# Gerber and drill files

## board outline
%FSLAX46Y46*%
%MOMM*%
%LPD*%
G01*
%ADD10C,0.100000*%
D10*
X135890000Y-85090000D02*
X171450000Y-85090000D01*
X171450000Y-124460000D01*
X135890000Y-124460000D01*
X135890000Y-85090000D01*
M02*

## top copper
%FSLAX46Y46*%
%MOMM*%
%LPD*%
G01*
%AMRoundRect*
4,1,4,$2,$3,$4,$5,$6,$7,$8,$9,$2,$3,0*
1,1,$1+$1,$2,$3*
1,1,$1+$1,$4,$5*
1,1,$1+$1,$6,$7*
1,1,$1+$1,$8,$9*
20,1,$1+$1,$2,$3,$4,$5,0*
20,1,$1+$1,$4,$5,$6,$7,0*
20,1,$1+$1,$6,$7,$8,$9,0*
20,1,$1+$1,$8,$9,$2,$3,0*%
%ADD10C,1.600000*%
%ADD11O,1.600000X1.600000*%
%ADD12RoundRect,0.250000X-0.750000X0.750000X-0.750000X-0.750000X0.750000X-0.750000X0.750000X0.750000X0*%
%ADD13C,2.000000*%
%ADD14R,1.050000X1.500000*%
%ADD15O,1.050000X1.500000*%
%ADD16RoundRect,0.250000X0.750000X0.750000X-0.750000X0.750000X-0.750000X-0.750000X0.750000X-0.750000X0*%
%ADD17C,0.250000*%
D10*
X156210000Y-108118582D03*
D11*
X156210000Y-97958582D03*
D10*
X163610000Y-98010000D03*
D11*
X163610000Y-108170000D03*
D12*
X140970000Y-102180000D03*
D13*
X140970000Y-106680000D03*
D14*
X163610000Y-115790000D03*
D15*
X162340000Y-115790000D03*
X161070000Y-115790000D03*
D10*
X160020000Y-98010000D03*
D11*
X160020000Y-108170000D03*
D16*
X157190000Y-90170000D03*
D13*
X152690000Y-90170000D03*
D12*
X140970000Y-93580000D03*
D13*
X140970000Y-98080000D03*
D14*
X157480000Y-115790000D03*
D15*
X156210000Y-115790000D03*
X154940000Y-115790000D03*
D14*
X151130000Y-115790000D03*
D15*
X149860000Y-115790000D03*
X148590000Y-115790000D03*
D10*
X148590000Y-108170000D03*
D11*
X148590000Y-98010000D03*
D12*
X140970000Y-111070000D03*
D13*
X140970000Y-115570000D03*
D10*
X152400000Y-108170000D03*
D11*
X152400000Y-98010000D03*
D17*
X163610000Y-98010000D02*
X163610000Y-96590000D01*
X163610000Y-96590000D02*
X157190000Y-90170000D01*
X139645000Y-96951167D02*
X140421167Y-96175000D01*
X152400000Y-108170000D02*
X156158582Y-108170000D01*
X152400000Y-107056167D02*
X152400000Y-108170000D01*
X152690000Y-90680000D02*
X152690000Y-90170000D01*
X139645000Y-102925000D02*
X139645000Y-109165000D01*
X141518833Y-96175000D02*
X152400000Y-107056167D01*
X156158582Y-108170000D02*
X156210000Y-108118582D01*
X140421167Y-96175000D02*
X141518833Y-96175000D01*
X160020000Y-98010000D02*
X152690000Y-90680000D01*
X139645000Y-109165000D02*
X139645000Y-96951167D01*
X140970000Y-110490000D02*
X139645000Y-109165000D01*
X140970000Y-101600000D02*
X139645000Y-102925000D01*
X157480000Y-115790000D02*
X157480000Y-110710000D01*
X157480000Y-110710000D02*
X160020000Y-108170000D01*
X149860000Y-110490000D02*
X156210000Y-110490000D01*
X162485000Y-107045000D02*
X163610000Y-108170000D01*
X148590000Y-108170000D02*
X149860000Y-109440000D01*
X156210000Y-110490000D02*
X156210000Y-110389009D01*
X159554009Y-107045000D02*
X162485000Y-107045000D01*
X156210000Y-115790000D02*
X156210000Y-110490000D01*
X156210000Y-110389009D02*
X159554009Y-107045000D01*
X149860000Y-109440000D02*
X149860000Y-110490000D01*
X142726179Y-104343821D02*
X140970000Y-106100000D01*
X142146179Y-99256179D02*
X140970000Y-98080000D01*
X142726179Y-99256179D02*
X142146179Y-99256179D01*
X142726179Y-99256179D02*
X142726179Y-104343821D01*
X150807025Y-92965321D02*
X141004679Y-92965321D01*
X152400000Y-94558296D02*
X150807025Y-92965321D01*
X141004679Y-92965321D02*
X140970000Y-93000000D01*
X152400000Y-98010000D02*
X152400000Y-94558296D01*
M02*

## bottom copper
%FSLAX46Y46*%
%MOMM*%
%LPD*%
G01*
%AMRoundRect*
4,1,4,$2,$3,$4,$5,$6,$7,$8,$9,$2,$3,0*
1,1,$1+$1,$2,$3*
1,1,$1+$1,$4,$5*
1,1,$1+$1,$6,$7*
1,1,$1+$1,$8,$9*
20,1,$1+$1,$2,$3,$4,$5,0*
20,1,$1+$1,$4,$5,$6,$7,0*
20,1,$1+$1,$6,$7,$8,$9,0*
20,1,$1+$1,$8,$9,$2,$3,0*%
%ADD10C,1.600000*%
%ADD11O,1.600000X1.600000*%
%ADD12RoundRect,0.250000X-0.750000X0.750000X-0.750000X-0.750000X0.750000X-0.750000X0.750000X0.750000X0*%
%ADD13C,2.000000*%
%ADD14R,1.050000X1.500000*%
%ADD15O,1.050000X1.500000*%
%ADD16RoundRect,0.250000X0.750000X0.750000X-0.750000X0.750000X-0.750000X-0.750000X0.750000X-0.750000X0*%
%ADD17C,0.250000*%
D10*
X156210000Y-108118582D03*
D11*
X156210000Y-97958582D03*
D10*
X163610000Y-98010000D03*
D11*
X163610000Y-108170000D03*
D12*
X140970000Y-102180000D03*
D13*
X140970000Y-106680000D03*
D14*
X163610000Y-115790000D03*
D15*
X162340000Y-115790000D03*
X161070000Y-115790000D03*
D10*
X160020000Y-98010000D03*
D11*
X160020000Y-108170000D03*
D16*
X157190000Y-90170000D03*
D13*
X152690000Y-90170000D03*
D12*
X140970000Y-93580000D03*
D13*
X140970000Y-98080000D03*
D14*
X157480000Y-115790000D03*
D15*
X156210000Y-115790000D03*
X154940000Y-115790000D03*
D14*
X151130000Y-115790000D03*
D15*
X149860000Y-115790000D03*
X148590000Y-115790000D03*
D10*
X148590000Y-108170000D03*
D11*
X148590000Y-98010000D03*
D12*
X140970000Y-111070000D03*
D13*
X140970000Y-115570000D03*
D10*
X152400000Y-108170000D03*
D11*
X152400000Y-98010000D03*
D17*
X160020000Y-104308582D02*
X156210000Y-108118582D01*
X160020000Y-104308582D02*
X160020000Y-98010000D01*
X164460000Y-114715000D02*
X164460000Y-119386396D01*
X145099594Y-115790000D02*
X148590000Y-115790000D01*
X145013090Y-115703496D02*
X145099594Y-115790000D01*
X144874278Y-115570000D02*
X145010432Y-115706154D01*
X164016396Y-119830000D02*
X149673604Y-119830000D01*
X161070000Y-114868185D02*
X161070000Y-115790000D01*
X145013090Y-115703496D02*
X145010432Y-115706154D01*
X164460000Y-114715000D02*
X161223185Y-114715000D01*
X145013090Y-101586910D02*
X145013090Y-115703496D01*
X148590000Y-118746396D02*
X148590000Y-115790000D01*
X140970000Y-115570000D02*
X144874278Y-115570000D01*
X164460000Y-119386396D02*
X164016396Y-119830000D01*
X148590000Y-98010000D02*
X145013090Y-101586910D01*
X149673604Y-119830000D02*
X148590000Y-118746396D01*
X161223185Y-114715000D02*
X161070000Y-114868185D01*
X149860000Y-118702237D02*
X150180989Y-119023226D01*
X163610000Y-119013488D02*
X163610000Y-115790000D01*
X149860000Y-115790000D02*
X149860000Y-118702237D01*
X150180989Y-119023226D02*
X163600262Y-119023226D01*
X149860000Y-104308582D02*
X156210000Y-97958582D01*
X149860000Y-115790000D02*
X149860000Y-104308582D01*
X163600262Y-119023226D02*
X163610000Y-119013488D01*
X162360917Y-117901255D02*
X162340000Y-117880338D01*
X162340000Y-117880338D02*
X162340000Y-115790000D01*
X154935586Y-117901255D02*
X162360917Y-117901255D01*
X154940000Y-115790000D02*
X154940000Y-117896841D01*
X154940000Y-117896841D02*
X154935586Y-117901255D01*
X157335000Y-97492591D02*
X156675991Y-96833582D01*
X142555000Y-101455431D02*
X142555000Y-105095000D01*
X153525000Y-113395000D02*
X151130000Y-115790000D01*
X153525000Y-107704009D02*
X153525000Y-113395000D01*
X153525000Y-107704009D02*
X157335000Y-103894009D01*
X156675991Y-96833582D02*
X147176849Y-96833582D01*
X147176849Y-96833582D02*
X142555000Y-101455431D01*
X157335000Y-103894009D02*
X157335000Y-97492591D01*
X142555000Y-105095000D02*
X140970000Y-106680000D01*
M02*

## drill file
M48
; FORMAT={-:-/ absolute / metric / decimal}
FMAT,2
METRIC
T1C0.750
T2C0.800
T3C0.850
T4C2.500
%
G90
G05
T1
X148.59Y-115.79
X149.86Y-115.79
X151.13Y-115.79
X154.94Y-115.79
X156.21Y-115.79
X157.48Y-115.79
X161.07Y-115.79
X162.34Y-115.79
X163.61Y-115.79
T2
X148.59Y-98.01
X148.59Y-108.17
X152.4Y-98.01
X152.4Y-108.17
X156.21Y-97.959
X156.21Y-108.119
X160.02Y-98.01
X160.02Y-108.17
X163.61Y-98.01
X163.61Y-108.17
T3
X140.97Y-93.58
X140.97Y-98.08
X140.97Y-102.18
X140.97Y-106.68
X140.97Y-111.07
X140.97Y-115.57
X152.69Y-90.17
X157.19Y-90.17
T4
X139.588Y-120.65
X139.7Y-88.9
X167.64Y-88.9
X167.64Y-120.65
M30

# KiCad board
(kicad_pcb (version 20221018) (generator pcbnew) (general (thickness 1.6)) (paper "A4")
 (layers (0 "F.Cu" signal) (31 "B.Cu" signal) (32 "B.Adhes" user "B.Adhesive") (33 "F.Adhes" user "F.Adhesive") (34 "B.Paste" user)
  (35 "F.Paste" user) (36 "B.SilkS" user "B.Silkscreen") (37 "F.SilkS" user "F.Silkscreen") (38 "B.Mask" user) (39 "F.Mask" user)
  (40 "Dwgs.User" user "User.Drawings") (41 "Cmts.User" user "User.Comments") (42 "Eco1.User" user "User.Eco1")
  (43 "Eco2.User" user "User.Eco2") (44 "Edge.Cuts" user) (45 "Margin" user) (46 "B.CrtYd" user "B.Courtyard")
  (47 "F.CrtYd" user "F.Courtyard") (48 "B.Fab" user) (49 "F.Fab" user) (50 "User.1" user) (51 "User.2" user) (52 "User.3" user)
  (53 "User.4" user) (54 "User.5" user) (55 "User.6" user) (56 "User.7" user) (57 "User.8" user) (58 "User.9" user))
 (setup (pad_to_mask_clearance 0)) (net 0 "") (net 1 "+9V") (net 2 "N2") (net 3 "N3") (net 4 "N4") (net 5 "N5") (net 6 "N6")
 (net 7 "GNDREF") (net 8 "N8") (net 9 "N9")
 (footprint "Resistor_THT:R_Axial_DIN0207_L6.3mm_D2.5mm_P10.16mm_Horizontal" (layer "F.Cu") (at 156.21 108.118582 90)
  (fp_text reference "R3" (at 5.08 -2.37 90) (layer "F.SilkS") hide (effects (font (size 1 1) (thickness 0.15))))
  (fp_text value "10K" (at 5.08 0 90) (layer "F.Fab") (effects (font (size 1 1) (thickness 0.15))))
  (pad "1" thru_hole circle (at 0 0 90) (size 1.6 1.6) (drill 0.8) (layers "*.Cu" "*.Mask") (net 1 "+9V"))
  (pad "2" thru_hole oval (at 10.16 0 90) (size 1.6 1.6) (drill 0.8) (layers "*.Cu" "*.Mask") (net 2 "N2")))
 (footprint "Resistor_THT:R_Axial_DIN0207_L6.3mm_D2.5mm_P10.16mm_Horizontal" (layer "F.Cu") (at 163.61 98.01 -90)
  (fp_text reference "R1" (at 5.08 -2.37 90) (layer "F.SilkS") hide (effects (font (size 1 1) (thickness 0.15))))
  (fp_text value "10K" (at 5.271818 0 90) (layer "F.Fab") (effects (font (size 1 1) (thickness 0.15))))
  (pad "1" thru_hole circle (at 0 0 270) (size 1.6 1.6) (drill 0.8) (layers "*.Cu" "*.Mask") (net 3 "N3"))
  (pad "2" thru_hole oval (at 10.16 0 270) (size 1.6 1.6) (drill 0.8) (layers "*.Cu" "*.Mask") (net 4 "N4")))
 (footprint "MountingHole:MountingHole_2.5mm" (layer "F.Cu") (at 139.7 88.9)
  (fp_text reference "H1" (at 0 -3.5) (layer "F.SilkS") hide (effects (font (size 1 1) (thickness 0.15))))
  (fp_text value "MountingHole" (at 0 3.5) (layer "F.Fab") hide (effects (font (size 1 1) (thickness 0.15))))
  (pad "" np_thru_hole circle (at 0 0) (size 2.5 2.5) (drill 2.5) (layers "*.Cu" "*.Mask")))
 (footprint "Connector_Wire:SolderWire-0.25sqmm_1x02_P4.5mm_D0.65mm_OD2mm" (layer "F.Cu") (at 140.97 102.18 -90)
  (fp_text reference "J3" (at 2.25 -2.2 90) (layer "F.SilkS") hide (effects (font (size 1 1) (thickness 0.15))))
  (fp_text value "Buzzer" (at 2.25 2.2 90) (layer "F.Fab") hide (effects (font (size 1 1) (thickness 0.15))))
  (pad "1" thru_hole roundrect (at 0 0 270) (size 2 2) (drill 0.85) (layers "*.Cu" "*.Mask") (roundrect_rratio 0.125) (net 1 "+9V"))
  (pad "2" thru_hole circle (at 4.5 0 270) (size 2 2) (drill 0.85) (layers "*.Cu" "*.Mask") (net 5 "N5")))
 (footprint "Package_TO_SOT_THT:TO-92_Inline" (layer "F.Cu") (at 163.61 115.79 180)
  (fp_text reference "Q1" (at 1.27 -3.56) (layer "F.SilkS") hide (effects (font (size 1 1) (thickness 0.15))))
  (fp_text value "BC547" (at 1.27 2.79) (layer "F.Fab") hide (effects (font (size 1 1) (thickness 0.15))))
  (pad "1" thru_hole rect (at 0 0 180) (size 1.05 1.5) (drill 0.75) (layers "*.Cu" "*.Mask") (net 2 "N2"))
  (pad "2" thru_hole oval (at 1.27 0 180) (size 1.05 1.5) (drill 0.75) (layers "*.Cu" "*.Mask") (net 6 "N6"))
  (pad "3" thru_hole oval (at 2.54 0 180) (size 1.05 1.5) (drill 0.75) (layers "*.Cu" "*.Mask") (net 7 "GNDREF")))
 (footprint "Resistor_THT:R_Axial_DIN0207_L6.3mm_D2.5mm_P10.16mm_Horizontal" (layer "F.Cu") (at 160.02 98.01 -90)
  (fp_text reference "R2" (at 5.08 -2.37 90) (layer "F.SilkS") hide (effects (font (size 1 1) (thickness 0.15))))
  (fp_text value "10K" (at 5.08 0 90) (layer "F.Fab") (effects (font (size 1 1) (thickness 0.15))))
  (pad "1" thru_hole circle (at 0 0 270) (size 1.6 1.6) (drill 0.8) (layers "*.Cu" "*.Mask") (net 1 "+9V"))
  (pad "2" thru_hole oval (at 10.16 0 270) (size 1.6 1.6) (drill 0.8) (layers "*.Cu" "*.Mask") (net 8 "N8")))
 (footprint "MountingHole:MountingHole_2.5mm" (layer "F.Cu") (at 139.588015 120.65)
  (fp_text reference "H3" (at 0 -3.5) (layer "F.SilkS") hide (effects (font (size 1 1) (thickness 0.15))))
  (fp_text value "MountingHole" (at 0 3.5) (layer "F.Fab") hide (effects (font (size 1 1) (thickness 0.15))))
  (pad "" np_thru_hole circle (at 0 0) (size 2.5 2.5) (drill 2.5) (layers "*.Cu" "*.Mask")))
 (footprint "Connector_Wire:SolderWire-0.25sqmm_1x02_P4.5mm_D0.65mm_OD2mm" (layer "F.Cu") (at 157.19 90.17 180)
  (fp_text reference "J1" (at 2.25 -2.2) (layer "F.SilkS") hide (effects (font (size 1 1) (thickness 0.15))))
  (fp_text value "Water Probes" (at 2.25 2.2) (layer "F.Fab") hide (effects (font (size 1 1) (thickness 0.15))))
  (pad "1" thru_hole roundrect (at 0 0 180) (size 2 2) (drill 0.85) (layers "*.Cu" "*.Mask") (roundrect_rratio 0.125) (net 3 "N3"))
  (pad "2" thru_hole circle (at 4.5 0 180) (size 2 2) (drill 0.85) (layers "*.Cu" "*.Mask") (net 1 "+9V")))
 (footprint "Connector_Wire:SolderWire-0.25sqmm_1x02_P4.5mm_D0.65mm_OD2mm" (layer "F.Cu") (at 140.97 93.58 -90)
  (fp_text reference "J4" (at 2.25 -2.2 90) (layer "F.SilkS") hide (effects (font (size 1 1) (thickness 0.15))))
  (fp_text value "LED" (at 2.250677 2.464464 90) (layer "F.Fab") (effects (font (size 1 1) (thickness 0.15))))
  (pad "1" thru_hole roundrect (at 0 0 270) (size 2 2) (drill 0.85) (layers "*.Cu" "*.Mask") (roundrect_rratio 0.125) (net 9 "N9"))
  (pad "2" thru_hole circle (at 4.5 0 270) (size 2 2) (drill 0.85) (layers "*.Cu" "*.Mask") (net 5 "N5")))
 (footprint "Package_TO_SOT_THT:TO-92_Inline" (layer "F.Cu") (at 157.48 115.79 180)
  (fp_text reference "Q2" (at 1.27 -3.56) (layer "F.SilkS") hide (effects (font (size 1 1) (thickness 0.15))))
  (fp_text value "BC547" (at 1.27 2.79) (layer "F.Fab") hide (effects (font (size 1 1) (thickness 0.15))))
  (pad "1" thru_hole rect (at 0 0 180) (size 1.05 1.5) (drill 0.75) (layers "*.Cu" "*.Mask") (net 8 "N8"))
  (pad "2" thru_hole oval (at 1.27 0 180) (size 1.05 1.5) (drill 0.75) (layers "*.Cu" "*.Mask") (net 4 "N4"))
  (pad "3" thru_hole oval (at 2.54 0 180) (size 1.05 1.5) (drill 0.75) (layers "*.Cu" "*.Mask") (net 6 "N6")))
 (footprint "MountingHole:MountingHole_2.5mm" (layer "F.Cu") (at 167.64 120.65)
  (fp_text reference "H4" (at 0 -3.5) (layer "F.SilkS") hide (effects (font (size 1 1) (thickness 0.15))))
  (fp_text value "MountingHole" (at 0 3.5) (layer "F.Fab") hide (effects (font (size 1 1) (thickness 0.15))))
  (pad "" np_thru_hole circle (at 0 0) (size 2.5 2.5) (drill 2.5) (layers "*.Cu" "*.Mask")))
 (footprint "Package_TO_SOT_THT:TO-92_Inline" (layer "F.Cu") (at 151.13 115.79 180)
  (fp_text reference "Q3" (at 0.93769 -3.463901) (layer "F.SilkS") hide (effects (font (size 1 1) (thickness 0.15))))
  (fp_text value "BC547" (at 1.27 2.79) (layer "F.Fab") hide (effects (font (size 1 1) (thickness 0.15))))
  (pad "1" thru_hole rect (at 0 0 180) (size 1.05 1.5) (drill 0.75) (layers "*.Cu" "*.Mask") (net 5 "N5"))
  (pad "2" thru_hole oval (at 1.27 0 180) (size 1.05 1.5) (drill 0.75) (layers "*.Cu" "*.Mask") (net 2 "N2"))
  (pad "3" thru_hole oval (at 2.54 0 180) (size 1.05 1.5) (drill 0.75) (layers "*.Cu" "*.Mask") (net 7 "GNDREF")))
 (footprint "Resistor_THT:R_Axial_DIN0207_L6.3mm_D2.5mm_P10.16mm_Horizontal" (layer "F.Cu") (at 148.59 108.17 90)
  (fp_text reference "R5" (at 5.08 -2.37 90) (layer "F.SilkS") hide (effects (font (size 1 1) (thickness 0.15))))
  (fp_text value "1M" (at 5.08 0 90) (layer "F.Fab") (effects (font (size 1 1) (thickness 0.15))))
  (pad "1" thru_hole circle (at 0 0 90) (size 1.6 1.6) (drill 0.8) (layers "*.Cu" "*.Mask") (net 4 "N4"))
  (pad "2" thru_hole oval (at 10.16 0 90) (size 1.6 1.6) (drill 0.8) (layers "*.Cu" "*.Mask") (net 7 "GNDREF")))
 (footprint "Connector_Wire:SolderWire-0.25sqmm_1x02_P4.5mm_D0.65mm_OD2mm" (layer "F.Cu") (at 140.97 111.07 -90)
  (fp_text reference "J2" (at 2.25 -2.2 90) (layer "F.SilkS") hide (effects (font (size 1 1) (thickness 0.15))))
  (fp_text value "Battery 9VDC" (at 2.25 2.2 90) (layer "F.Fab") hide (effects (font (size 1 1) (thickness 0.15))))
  (pad "1" thru_hole roundrect (at 0 0 270) (size 2 2) (drill 0.85) (layers "*.Cu" "*.Mask") (roundrect_rratio 0.125) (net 1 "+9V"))
  (pad "2" thru_hole circle (at 4.5 0 270) (size 2 2) (drill 0.85) (layers "*.Cu" "*.Mask") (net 7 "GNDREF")))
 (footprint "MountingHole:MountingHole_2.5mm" (layer "F.Cu") (at 167.64 88.9)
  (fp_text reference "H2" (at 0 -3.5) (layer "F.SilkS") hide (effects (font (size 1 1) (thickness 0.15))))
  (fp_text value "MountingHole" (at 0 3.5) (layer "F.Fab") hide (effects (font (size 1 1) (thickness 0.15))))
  (pad "" np_thru_hole circle (at 0 0) (size 2.5 2.5) (drill 2.5) (layers "*.Cu" "*.Mask")))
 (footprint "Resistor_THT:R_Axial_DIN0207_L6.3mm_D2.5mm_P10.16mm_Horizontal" (layer "F.Cu") (at 152.4 108.17 90)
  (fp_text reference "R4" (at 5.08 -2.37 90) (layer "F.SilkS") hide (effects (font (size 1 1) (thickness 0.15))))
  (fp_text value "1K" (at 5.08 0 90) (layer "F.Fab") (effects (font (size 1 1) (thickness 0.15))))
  (pad "1" thru_hole circle (at 0 0 90) (size 1.6 1.6) (drill 0.8) (layers "*.Cu" "*.Mask") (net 1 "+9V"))
  (pad "2" thru_hole oval (at 10.16 0 90) (size 1.6 1.6) (drill 0.8) (layers "*.Cu" "*.Mask") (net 9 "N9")))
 (gr_rect (start 135.89 85.09) (end 171.45 124.46) (stroke (width 0.1) (type default)) (fill none) (layer "Edge.Cuts"))
 (segment (start 163.61 98.01) (end 163.61 96.59) (width 0.25) (layer "F.Cu") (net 3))
 (segment (start 163.61 96.59) (end 157.19 90.17) (width 0.25) (layer "F.Cu") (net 3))
 (segment (start 139.645 96.951167) (end 140.421167 96.175) (width 0.25) (layer "F.Cu") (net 1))
 (segment (start 152.4 108.17) (end 156.158582 108.17) (width 0.25) (layer "F.Cu") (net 1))
 (segment (start 152.4 107.056167) (end 152.4 108.17) (width 0.25) (layer "F.Cu") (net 1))
 (segment (start 152.69 90.68) (end 152.69 90.17) (width 0.25) (layer "F.Cu") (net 1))
 (segment (start 139.645 102.925) (end 139.645 109.165) (width 0.25) (layer "F.Cu") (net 1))
 (segment (start 141.518833 96.175) (end 152.4 107.056167) (width 0.25) (layer "F.Cu") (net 1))
 (segment (start 156.158582 108.17) (end 156.21 108.118582) (width 0.25) (layer "F.Cu") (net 1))
 (segment (start 140.421167 96.175) (end 141.518833 96.175) (width 0.25) (layer "F.Cu") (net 1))
 (segment (start 160.02 98.01) (end 152.69 90.68) (width 0.25) (layer "F.Cu") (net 1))
 (segment (start 139.645 109.165) (end 139.645 96.951167) (width 0.25) (layer "F.Cu") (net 1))
 (segment (start 140.97 110.49) (end 139.645 109.165) (width 0.25) (layer "F.Cu") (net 1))
 (segment (start 140.97 101.6) (end 139.645 102.925) (width 0.25) (layer "F.Cu") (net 1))
 (segment (start 160.02 104.308582) (end 156.21 108.118582) (width 0.25) (layer "B.Cu") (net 1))
 (segment (start 160.02 104.308582) (end 160.02 98.01) (width 0.25) (layer "B.Cu") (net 1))
 (segment (start 164.46 114.715) (end 164.46 119.386396) (width 0.25) (layer "B.Cu") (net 7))
 (segment (start 145.099594 115.79) (end 148.59 115.79) (width 0.25) (layer "B.Cu") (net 7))
 (segment (start 145.01309 115.703496) (end 145.099594 115.79) (width 0.25) (layer "B.Cu") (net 7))
 (segment (start 144.874278 115.57) (end 145.010432 115.706154) (width 0.25) (layer "B.Cu") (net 7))
 (segment (start 164.016396 119.83) (end 149.673604 119.83) (width 0.25) (layer "B.Cu") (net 7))
 (segment (start 161.07 114.868185) (end 161.07 115.79) (width 0.25) (layer "B.Cu") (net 7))
 (segment (start 145.01309 115.703496) (end 145.010432 115.706154) (width 0.25) (layer "B.Cu") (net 7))
 (segment (start 164.46 114.715) (end 161.223185 114.715) (width 0.25) (layer "B.Cu") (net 7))
 (segment (start 145.01309 101.58691) (end 145.01309 115.703496) (width 0.25) (layer "B.Cu") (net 7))
 (segment (start 148.59 118.746396) (end 148.59 115.79) (width 0.25) (layer "B.Cu") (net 7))
 (segment (start 140.97 115.57) (end 144.874278 115.57) (width 0.25) (layer "B.Cu") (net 7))
 (segment (start 164.46 119.386396) (end 164.016396 119.83) (width 0.25) (layer "B.Cu") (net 7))
 (segment (start 148.59 98.01) (end 145.01309 101.58691) (width 0.25) (layer "B.Cu") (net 7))
 (segment (start 149.673604 119.83) (end 148.59 118.746396) (width 0.25) (layer "B.Cu") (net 7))
 (segment (start 161.223185 114.715) (end 161.07 114.868185) (width 0.25) (layer "B.Cu") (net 7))
 (segment (start 149.86 118.702237) (end 150.180989 119.023226) (width 0.25) (layer "B.Cu") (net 2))
 (segment (start 163.61 119.013488) (end 163.61 115.79) (width 0.25) (layer "B.Cu") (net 2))
 (segment (start 149.86 115.79) (end 149.86 118.702237) (width 0.25) (layer "B.Cu") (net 2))
 (segment (start 150.180989 119.023226) (end 163.600262 119.023226) (width 0.25) (layer "B.Cu") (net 2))
 (segment (start 149.86 104.308582) (end 156.21 97.958582) (width 0.25) (layer "B.Cu") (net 2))
 (segment (start 149.86 115.79) (end 149.86 104.308582) (width 0.25) (layer "B.Cu") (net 2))
 (segment (start 163.600262 119.023226) (end 163.61 119.013488) (width 0.25) (layer "B.Cu") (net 2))
 (segment (start 162.360917 117.901255) (end 162.34 117.880338) (width 0.25) (layer "B.Cu") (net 6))
 (segment (start 162.34 117.880338) (end 162.34 115.79) (width 0.25) (layer "B.Cu") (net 6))
 (segment (start 154.935586 117.901255) (end 162.360917 117.901255) (width 0.25) (layer "B.Cu") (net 6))
 (segment (start 154.94 115.79) (end 154.94 117.896841) (width 0.25) (layer "B.Cu") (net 6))
 (segment (start 154.94 117.896841) (end 154.935586 117.901255) (width 0.25) (layer "B.Cu") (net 6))
 (segment (start 157.48 115.79) (end 157.48 110.71) (width 0.25) (layer "F.Cu") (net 8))
 (segment (start 157.48 110.71) (end 160.02 108.17) (width 0.25) (layer "F.Cu") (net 8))
 (segment (start 149.86 110.49) (end 156.21 110.49) (width 0.25) (layer "F.Cu") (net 4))
 (segment (start 162.485 107.045) (end 163.61 108.17) (width 0.25) (layer "F.Cu") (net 4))
 (segment (start 148.59 108.17) (end 149.86 109.44) (width 0.25) (layer "F.Cu") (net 4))
 (segment (start 156.21 110.49) (end 156.21 110.389009) (width 0.25) (layer "F.Cu") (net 4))
 (segment (start 159.554009 107.045) (end 162.485 107.045) (width 0.25) (layer "F.Cu") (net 4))
 (segment (start 156.21 115.79) (end 156.21 110.49) (width 0.25) (layer "F.Cu") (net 4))
 (segment (start 156.21 110.389009) (end 159.554009 107.045) (width 0.25) (layer "F.Cu") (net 4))
 (segment (start 149.86 109.44) (end 149.86 110.49) (width 0.25) (layer "F.Cu") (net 4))
 (segment (start 142.726179 104.343821) (end 140.97 106.1) (width 0.25) (layer "F.Cu") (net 5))
 (segment (start 142.146179 99.256179) (end 140.97 98.08) (width 0.25) (layer "F.Cu") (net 5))
 (segment (start 142.726179 99.256179) (end 142.146179 99.256179) (width 0.25) (layer "F.Cu") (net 5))
 (segment (start 142.726179 99.256179) (end 142.726179 104.343821) (width 0.25) (layer "F.Cu") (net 5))
 (segment (start 157.335 97.492591) (end 156.675991 96.833582) (width 0.25) (layer "B.Cu") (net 5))
 (segment (start 142.555 101.455431) (end 142.555 105.095) (width 0.25) (layer "B.Cu") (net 5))
 (segment (start 153.525 113.395) (end 151.13 115.79) (width 0.25) (layer "B.Cu") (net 5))
 (segment (start 153.525 107.704009) (end 153.525 113.395) (width 0.25) (layer "B.Cu") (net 5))
 (segment (start 153.525 107.704009) (end 157.335 103.894009) (width 0.25) (layer "B.Cu") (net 5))
 (segment (start 156.675991 96.833582) (end 147.176849 96.833582) (width 0.25) (layer "B.Cu") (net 5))
 (segment (start 147.176849 96.833582) (end 142.555 101.455431) (width 0.25) (layer "B.Cu") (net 5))
 (segment (start 157.335 103.894009) (end 157.335 97.492591) (width 0.25) (layer "B.Cu") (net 5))
 (segment (start 142.555 105.095) (end 140.97 106.68) (width 0.25) (layer "B.Cu") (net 5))
 (segment (start 150.807025 92.965321) (end 141.004679 92.965321) (width 0.25) (layer "F.Cu") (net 9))
 (segment (start 152.4 94.558296) (end 150.807025 92.965321) (width 0.25) (layer "F.Cu") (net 9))
 (segment (start 141.004679 92.965321) (end 140.97 93) (width 0.25) (layer "F.Cu") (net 9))
 (segment (start 152.4 98.01) (end 152.4 94.558296) (width 0.25) (layer "F.Cu") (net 9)))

